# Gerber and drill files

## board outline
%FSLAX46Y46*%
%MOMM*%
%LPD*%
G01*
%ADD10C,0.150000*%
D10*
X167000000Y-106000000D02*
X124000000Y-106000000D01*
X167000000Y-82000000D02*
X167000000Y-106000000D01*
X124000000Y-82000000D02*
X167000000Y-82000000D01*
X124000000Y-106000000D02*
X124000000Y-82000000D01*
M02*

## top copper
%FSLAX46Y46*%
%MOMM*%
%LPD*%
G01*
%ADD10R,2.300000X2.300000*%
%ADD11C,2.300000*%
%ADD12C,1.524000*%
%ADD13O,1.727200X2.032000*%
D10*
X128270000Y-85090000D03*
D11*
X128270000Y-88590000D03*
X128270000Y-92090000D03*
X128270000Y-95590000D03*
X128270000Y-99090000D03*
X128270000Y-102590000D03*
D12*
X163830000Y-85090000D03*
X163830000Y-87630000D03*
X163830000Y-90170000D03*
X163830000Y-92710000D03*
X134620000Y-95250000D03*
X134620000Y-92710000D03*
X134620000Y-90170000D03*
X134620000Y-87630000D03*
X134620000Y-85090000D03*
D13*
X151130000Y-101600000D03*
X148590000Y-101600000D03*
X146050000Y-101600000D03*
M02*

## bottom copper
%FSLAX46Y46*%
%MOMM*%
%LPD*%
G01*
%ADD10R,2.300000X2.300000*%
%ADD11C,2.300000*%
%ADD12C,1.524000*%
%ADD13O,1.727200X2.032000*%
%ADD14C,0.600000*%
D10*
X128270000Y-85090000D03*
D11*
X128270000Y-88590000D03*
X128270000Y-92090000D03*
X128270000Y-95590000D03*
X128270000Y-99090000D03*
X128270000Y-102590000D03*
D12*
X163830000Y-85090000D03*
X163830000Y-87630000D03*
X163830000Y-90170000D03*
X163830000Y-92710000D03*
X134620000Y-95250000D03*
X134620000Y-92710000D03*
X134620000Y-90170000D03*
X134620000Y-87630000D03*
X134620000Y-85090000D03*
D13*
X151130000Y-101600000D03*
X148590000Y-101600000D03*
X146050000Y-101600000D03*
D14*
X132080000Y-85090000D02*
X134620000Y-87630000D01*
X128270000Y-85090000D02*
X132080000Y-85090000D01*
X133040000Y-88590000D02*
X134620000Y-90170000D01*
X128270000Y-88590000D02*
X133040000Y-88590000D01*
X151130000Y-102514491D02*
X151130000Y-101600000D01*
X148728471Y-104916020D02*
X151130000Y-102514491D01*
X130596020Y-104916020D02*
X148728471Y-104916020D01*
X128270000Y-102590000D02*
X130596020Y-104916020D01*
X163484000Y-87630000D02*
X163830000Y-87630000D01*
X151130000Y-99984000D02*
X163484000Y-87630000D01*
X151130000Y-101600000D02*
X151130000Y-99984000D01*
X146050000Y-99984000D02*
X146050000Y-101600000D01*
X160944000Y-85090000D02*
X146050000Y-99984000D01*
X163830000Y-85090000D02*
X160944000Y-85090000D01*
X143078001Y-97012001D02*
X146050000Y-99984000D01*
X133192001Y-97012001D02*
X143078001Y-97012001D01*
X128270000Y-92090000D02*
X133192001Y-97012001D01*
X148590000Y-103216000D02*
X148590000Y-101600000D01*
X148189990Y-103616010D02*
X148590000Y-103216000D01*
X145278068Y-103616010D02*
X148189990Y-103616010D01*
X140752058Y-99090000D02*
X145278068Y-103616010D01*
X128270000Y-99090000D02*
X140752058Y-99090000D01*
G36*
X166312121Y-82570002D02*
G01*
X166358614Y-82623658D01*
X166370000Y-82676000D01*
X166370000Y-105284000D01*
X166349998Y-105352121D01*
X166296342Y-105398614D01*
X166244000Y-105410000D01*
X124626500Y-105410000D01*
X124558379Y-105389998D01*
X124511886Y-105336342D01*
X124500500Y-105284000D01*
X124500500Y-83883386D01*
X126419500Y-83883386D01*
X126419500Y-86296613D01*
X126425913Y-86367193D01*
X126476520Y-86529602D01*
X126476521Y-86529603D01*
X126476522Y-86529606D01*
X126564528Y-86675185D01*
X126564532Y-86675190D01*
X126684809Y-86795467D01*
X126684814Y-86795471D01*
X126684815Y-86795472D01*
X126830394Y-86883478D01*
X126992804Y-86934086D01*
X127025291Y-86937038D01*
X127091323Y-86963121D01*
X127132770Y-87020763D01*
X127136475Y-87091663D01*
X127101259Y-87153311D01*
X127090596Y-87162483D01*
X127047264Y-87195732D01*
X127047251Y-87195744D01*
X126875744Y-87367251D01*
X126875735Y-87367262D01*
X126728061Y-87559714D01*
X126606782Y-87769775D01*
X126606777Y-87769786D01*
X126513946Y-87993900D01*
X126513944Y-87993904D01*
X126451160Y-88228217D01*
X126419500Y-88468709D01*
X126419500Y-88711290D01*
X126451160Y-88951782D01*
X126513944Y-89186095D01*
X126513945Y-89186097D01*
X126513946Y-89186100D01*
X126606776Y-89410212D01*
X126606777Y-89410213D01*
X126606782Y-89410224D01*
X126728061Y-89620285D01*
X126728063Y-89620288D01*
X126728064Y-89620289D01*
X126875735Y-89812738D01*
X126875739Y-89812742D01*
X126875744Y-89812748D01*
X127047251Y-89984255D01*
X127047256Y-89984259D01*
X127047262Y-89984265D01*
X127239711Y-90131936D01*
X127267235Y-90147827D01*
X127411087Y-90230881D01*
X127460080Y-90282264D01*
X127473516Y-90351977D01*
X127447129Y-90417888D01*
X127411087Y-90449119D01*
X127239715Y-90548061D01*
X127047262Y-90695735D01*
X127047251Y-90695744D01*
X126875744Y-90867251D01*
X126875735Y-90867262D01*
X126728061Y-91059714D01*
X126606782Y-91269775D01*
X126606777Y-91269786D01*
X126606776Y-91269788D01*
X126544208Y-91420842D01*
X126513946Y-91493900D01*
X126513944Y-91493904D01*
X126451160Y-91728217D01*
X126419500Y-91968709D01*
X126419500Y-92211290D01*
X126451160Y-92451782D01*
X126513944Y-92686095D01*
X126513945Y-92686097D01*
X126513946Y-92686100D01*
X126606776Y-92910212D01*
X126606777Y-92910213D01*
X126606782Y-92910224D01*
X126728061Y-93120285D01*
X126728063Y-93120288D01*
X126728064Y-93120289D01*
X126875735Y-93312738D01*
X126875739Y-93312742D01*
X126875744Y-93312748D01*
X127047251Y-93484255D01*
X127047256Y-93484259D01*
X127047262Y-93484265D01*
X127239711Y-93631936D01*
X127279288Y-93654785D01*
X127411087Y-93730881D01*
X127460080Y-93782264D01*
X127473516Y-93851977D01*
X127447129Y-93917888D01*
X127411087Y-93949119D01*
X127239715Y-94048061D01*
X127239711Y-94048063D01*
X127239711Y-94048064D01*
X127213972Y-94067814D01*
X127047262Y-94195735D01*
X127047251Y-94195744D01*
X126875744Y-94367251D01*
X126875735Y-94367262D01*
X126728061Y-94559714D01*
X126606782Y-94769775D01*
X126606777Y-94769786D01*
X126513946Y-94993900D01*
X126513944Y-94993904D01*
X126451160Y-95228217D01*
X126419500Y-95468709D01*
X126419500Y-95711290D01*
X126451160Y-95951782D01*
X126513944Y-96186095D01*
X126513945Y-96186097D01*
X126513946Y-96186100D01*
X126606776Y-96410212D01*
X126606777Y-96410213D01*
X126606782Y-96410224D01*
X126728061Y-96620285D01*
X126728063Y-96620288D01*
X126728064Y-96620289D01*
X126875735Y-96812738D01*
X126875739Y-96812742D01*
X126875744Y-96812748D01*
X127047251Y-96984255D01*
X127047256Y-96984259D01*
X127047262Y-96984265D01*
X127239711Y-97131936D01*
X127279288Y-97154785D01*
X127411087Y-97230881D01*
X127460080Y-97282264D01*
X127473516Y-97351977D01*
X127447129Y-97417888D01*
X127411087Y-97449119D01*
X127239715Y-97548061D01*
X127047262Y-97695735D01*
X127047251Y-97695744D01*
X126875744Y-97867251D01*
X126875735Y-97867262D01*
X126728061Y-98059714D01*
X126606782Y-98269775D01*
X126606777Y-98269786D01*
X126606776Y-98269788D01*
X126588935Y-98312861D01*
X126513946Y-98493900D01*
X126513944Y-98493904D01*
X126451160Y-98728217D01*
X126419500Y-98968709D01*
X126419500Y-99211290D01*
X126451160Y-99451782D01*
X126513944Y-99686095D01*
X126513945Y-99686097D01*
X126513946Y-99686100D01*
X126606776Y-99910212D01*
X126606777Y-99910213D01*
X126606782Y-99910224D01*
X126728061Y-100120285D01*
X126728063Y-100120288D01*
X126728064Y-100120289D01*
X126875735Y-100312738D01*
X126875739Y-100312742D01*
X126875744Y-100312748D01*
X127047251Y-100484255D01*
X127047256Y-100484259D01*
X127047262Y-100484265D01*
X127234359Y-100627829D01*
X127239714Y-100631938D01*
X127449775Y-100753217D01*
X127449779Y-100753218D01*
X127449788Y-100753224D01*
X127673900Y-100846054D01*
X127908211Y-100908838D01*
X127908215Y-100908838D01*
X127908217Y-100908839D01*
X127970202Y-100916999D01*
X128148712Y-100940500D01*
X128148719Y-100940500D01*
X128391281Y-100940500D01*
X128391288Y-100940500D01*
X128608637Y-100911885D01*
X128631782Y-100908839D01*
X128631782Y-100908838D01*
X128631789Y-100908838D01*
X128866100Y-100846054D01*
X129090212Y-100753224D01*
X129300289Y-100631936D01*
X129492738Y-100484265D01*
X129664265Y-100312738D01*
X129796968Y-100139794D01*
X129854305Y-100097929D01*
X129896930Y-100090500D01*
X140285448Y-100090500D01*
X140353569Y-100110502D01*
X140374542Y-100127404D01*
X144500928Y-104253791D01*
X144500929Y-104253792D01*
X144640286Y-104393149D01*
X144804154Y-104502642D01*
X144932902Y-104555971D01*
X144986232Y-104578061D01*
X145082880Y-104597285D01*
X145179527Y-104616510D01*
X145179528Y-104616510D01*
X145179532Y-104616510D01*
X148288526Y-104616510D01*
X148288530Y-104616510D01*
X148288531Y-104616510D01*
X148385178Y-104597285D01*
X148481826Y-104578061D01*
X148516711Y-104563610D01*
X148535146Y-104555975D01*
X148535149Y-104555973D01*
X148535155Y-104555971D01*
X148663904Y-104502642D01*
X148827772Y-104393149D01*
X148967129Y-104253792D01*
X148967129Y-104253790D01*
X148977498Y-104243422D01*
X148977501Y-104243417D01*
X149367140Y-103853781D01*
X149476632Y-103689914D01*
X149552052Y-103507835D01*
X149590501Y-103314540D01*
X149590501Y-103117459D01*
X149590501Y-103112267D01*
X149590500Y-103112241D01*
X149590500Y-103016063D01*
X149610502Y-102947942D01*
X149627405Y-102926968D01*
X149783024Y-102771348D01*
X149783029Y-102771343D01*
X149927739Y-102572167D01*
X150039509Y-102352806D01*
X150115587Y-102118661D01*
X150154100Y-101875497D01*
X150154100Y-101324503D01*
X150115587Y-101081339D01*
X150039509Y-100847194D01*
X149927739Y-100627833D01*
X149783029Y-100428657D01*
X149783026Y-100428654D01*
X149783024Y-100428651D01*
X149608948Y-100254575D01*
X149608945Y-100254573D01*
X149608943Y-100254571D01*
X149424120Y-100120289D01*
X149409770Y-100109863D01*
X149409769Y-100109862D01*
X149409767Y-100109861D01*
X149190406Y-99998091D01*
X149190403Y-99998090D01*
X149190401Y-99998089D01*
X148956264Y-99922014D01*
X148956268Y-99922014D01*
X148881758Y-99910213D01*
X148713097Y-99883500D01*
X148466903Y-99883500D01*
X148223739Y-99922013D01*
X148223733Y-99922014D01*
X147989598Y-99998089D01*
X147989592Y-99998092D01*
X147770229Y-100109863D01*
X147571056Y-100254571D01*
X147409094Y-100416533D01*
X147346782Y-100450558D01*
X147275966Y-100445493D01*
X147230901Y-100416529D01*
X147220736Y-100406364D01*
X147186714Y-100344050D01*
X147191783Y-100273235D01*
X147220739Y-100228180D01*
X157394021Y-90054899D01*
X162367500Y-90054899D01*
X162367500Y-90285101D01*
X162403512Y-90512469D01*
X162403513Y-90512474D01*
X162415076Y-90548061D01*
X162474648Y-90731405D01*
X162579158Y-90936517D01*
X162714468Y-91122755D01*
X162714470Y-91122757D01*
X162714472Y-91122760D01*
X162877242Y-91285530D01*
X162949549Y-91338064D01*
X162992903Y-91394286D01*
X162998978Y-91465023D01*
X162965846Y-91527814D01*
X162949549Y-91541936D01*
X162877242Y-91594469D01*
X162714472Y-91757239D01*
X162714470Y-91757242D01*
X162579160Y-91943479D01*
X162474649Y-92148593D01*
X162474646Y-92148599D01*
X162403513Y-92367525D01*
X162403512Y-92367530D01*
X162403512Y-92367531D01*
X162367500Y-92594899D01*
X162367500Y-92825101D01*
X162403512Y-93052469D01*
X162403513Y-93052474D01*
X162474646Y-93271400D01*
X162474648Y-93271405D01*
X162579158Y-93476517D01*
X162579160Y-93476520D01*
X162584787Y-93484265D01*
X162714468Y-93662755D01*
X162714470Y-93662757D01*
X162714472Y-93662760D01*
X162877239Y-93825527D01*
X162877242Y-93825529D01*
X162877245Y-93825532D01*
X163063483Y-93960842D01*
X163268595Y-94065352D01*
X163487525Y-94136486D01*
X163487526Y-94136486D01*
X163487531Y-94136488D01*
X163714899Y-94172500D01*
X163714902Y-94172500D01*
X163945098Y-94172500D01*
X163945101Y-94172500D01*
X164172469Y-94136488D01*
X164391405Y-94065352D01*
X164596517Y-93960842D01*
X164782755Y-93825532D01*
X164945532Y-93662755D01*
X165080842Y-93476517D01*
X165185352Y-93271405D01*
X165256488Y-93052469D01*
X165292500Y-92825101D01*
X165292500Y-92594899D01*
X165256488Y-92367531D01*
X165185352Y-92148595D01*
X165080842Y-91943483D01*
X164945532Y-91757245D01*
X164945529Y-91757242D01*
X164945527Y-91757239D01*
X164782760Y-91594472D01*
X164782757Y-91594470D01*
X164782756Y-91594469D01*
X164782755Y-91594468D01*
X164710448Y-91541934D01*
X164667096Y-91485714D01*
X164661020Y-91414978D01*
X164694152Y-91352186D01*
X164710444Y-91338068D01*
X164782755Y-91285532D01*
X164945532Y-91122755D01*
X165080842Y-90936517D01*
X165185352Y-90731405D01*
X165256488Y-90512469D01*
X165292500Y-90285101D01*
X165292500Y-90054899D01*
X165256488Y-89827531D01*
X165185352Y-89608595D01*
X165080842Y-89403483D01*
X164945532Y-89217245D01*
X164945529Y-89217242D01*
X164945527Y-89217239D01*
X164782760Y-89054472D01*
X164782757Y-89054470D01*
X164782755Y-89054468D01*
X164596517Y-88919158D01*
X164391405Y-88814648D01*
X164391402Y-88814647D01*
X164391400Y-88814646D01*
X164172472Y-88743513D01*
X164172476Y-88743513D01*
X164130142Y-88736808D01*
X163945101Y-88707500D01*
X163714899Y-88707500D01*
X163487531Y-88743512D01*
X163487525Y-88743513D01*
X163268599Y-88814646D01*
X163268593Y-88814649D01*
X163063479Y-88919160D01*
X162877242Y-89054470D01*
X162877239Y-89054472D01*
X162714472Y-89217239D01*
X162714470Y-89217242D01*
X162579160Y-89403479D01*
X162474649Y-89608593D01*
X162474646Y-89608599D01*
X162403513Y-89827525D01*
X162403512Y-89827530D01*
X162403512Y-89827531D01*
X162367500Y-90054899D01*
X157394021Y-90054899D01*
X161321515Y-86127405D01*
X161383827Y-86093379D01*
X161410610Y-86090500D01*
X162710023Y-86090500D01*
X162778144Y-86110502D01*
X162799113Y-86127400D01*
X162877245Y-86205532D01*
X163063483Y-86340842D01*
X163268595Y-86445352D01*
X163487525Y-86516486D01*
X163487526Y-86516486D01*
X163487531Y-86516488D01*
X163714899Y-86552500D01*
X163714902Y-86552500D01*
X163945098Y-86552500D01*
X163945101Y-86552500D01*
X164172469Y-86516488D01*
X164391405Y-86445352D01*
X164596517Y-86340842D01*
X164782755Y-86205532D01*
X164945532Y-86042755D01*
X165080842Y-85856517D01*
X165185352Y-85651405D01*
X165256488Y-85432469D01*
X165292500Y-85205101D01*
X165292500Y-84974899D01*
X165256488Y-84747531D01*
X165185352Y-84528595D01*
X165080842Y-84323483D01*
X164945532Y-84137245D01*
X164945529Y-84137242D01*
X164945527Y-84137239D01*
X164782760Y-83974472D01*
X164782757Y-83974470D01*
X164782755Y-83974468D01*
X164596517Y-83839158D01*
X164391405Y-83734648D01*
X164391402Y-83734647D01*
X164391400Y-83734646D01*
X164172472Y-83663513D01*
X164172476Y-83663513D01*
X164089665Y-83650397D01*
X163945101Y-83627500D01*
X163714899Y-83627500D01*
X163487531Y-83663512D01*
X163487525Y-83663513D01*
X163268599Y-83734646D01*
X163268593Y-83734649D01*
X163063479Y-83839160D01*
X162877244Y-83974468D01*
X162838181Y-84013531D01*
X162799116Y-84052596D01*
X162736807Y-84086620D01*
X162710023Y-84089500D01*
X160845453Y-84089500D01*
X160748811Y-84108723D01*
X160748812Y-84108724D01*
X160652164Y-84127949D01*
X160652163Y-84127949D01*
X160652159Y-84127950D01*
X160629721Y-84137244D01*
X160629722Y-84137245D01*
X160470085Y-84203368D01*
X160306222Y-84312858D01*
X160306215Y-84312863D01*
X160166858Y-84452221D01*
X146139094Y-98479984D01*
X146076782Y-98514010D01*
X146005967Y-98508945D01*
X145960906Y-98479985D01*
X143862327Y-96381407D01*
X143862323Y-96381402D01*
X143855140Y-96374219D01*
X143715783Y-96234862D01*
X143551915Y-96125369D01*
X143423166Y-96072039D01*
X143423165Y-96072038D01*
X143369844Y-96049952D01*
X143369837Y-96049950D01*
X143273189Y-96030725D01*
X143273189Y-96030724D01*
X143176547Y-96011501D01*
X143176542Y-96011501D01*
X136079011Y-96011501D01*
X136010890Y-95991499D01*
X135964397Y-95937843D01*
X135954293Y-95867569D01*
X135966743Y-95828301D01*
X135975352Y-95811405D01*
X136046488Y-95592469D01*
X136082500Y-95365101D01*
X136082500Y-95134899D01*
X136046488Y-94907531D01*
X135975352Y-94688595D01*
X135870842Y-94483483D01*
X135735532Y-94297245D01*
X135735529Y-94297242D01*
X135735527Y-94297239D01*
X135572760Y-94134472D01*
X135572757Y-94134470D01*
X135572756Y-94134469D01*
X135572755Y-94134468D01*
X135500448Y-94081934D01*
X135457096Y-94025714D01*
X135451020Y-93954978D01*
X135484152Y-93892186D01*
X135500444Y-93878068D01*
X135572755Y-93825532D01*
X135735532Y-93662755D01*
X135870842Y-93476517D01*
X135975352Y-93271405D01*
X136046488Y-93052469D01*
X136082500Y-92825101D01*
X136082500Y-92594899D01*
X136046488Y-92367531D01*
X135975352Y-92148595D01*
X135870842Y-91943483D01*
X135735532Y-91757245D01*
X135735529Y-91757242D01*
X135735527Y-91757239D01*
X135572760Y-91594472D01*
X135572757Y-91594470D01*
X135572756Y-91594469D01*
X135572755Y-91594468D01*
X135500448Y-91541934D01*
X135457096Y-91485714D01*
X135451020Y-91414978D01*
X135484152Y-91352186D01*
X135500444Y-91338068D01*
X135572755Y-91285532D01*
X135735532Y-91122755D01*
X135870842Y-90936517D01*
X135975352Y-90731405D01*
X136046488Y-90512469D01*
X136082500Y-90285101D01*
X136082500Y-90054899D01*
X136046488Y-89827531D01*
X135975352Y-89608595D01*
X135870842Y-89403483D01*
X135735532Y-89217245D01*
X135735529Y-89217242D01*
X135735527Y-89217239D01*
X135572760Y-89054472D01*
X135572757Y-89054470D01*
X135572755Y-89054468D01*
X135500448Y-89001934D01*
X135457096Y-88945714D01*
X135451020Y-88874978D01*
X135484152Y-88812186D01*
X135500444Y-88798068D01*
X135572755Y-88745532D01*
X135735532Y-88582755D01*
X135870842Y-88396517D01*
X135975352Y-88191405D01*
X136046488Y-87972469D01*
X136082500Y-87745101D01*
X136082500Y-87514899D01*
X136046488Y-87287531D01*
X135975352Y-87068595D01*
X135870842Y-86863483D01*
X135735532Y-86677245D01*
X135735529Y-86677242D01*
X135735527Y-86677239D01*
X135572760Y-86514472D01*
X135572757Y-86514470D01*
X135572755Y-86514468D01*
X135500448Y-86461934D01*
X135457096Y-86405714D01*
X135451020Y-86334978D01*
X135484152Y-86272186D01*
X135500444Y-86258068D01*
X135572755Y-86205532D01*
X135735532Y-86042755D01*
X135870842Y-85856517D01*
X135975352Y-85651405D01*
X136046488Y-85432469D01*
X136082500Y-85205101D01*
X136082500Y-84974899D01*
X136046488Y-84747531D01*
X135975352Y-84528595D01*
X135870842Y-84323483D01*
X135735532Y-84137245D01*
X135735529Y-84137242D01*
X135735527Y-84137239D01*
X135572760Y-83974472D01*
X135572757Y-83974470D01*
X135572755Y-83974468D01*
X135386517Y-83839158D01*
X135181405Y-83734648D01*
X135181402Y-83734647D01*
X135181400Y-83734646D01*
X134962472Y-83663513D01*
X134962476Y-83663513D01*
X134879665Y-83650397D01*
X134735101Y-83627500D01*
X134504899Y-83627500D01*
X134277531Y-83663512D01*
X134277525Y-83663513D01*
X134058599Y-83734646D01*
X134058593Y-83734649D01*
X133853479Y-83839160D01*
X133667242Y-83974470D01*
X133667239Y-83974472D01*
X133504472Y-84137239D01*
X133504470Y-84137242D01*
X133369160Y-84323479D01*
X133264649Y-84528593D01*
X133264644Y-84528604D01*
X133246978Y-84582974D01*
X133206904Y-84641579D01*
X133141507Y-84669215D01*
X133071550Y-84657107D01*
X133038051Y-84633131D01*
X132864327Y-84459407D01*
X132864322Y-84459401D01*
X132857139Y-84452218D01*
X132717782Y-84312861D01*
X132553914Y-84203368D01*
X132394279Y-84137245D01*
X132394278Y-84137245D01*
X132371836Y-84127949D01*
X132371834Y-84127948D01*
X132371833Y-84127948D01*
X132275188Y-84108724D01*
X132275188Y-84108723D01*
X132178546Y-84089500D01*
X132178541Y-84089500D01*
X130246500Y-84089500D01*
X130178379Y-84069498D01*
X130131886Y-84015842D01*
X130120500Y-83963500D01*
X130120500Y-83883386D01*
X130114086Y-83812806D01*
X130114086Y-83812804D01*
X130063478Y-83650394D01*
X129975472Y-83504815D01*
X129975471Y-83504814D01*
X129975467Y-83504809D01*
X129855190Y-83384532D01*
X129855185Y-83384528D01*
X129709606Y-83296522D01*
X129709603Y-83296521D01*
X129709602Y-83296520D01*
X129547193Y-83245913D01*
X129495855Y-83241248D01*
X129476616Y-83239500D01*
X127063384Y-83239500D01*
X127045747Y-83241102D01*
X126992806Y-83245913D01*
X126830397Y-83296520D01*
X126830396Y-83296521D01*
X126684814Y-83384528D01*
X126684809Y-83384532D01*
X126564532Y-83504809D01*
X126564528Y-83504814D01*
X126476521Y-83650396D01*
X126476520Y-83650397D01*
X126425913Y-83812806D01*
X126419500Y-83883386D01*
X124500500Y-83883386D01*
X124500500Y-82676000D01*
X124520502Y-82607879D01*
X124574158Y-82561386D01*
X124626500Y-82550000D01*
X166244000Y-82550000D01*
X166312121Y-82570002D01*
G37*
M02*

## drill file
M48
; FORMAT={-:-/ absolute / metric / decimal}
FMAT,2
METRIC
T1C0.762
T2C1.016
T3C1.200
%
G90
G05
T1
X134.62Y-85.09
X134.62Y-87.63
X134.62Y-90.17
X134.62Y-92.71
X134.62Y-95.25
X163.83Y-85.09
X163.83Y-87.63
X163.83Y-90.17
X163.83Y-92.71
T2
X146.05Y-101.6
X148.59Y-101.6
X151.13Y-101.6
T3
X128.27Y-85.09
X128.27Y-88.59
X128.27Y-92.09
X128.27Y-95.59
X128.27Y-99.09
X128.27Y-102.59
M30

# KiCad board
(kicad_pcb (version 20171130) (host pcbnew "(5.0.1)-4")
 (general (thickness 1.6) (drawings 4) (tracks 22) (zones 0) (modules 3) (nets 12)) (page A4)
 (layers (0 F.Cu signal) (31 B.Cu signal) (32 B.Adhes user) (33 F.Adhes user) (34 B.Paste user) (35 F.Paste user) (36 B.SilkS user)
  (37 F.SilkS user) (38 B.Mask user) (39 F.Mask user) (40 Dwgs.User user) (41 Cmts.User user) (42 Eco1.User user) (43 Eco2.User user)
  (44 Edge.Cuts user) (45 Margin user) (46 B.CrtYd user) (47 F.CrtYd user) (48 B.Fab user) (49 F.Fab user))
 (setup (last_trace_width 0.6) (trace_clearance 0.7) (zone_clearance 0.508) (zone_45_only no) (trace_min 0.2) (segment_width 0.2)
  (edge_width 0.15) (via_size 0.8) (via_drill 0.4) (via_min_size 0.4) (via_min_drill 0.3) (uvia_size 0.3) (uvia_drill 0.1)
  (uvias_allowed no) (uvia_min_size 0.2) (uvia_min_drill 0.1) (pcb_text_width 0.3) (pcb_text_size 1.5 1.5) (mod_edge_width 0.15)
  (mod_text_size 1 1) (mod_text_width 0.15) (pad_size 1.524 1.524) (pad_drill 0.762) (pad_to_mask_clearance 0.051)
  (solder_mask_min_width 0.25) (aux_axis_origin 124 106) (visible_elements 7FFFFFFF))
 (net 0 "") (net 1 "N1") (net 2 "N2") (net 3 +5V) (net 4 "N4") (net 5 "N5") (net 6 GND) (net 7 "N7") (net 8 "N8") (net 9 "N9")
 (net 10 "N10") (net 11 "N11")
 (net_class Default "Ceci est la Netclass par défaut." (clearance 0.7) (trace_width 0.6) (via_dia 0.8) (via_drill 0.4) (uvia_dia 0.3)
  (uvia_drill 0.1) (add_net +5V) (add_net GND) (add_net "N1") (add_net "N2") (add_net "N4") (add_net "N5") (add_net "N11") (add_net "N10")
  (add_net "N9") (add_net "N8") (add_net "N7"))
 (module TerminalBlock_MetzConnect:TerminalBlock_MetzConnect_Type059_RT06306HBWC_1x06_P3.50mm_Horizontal (layer F.Cu) (at 128.27 85.09 270)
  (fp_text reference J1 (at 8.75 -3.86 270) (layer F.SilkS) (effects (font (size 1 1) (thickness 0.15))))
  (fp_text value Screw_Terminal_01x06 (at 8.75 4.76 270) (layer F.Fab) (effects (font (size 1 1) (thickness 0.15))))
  (pad 1 thru_hole rect (at 0 0 270) (size 2.3 2.3) (drill 1.2) (layers *.Cu *.Mask) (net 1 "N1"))
  (pad 2 thru_hole circle (at 3.5 0 270) (size 2.3 2.3) (drill 1.2) (layers *.Cu *.Mask) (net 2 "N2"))
  (pad 3 thru_hole circle (at 7 0 270) (size 2.3 2.3) (drill 1.2) (layers *.Cu *.Mask) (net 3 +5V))
  (pad 4 thru_hole circle (at 10.5 0 270) (size 2.3 2.3) (drill 1.2) (layers *.Cu *.Mask) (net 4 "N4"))
  (pad 5 thru_hole circle (at 14 0 270) (size 2.3 2.3) (drill 1.2) (layers *.Cu *.Mask) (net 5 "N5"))
  (pad 6 thru_hole circle (at 17.5 0 270) (size 2.3 2.3) (drill 1.2) (layers *.Cu *.Mask) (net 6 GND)))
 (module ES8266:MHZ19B (layer F.Cu) (at 134.62 85.09)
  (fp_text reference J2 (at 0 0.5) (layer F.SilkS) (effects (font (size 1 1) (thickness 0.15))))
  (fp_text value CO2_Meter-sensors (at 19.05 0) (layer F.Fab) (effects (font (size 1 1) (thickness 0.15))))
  (pad 9 thru_hole circle (at 29.21 0) (size 1.524 1.524) (drill 0.762) (layers *.Cu *.Mask) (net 3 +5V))
  (pad 8 thru_hole circle (at 29.21 2.54) (size 1.524 1.524) (drill 0.762) (layers *.Cu *.Mask) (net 6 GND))
  (pad 7 thru_hole circle (at 29.21 5.08) (size 1.524 1.524) (drill 0.762) (layers *.Cu *.Mask) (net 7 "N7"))
  (pad 6 thru_hole circle (at 29.21 7.62) (size 1.524 1.524) (drill 0.762) (layers *.Cu *.Mask) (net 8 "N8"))
  (pad 5 thru_hole circle (at 0 10.16) (size 1.524 1.524) (drill 0.762) (layers *.Cu *.Mask) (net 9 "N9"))
  (pad 4 thru_hole circle (at 0 7.62) (size 1.524 1.524) (drill 0.762) (layers *.Cu *.Mask) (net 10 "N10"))
  (pad 3 thru_hole circle (at 0 5.08) (size 1.524 1.524) (drill 0.762) (layers *.Cu *.Mask) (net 2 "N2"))
  (pad 2 thru_hole circle (at 0 2.54) (size 1.524 1.524) (drill 0.762) (layers *.Cu *.Mask) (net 1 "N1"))
  (pad 1 thru_hole circle (at 0 0) (size 1.524 1.524) (drill 0.762) (layers *.Cu *.Mask) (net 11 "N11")))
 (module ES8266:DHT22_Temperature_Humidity (layer F.Cu) (at 148.59 101.6)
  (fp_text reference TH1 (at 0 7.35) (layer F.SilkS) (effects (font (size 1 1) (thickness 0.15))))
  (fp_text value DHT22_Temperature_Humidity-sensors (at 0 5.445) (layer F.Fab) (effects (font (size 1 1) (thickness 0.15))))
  (pad 3 thru_hole oval (at 2.54 0 90) (size 2.032 1.7272) (drill 1.016) (layers *.Cu *.Mask F.SilkS) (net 6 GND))
  (pad 2 thru_hole oval (at 0 0 90) (size 2.032 1.7272) (drill 1.016) (layers *.Cu *.Mask F.SilkS) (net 5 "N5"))
  (pad 1 thru_hole oval (at -2.54 0 90) (size 2.032 1.7272) (drill 1.016) (layers *.Cu *.Mask F.SilkS) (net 3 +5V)))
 (gr_line (start 167 106) (end 124 106) (layer Edge.Cuts) (width 0.15))
 (gr_line (start 167 82) (end 167 106) (layer Edge.Cuts) (width 0.15))
 (gr_line (start 124 82) (end 167 82) (layer Edge.Cuts) (width 0.15))
 (gr_line (start 124 106) (end 124 82) (layer Edge.Cuts) (width 0.15))
 (segment (start 132.08 85.09) (end 134.62 87.63) (width 0.6) (layer B.Cu) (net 1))
 (segment (start 128.27 85.09) (end 132.08 85.09) (width 0.6) (layer B.Cu) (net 1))
 (segment (start 133.04 88.59) (end 134.62 90.17) (width 0.6) (layer B.Cu) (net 2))
 (segment (start 128.27 88.59) (end 133.04 88.59) (width 0.6) (layer B.Cu) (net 2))
 (segment (start 151.13 102.514491) (end 151.13 101.6) (width 0.6) (layer B.Cu) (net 6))
 (segment (start 148.728471 104.91602) (end 151.13 102.514491) (width 0.6) (layer B.Cu) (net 6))
 (segment (start 130.59602 104.91602) (end 148.728471 104.91602) (width 0.6) (layer B.Cu) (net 6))
 (segment (start 128.27 102.59) (end 130.59602 104.91602) (width 0.6) (layer B.Cu) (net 6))
 (segment (start 163.484 87.63) (end 163.83 87.63) (width 0.6) (layer B.Cu) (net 6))
 (segment (start 151.13 99.984) (end 163.484 87.63) (width 0.6) (layer B.Cu) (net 6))
 (segment (start 151.13 101.6) (end 151.13 99.984) (width 0.6) (layer B.Cu) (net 6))
 (segment (start 146.05 99.984) (end 146.05 101.6) (width 0.6) (layer B.Cu) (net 3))
 (segment (start 160.944 85.09) (end 146.05 99.984) (width 0.6) (layer B.Cu) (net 3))
 (segment (start 163.83 85.09) (end 160.944 85.09) (width 0.6) (layer B.Cu) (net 3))
 (segment (start 143.078001 97.012001) (end 146.05 99.984) (width 0.6) (layer B.Cu) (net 3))
 (segment (start 133.192001 97.012001) (end 143.078001 97.012001) (width 0.6) (layer B.Cu) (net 3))
 (segment (start 128.27 92.09) (end 133.192001 97.012001) (width 0.6) (layer B.Cu) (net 3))
 (segment (start 148.59 103.216) (end 148.59 101.6) (width 0.6) (layer B.Cu) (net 5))
 (segment (start 148.18999 103.61601) (end 148.59 103.216) (width 0.6) (layer B.Cu) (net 5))
 (segment (start 145.278068 103.61601) (end 148.18999 103.61601) (width 0.6) (layer B.Cu) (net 5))
 (segment (start 140.752058 99.09) (end 145.278068 103.61601) (width 0.6) (layer B.Cu) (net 5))
 (segment (start 128.27 99.09) (end 140.752058 99.09) (width 0.6) (layer B.Cu) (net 5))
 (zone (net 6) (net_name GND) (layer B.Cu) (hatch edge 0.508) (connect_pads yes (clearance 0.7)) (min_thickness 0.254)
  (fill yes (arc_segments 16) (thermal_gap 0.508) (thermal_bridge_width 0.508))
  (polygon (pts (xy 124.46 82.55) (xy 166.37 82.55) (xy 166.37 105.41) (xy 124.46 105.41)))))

